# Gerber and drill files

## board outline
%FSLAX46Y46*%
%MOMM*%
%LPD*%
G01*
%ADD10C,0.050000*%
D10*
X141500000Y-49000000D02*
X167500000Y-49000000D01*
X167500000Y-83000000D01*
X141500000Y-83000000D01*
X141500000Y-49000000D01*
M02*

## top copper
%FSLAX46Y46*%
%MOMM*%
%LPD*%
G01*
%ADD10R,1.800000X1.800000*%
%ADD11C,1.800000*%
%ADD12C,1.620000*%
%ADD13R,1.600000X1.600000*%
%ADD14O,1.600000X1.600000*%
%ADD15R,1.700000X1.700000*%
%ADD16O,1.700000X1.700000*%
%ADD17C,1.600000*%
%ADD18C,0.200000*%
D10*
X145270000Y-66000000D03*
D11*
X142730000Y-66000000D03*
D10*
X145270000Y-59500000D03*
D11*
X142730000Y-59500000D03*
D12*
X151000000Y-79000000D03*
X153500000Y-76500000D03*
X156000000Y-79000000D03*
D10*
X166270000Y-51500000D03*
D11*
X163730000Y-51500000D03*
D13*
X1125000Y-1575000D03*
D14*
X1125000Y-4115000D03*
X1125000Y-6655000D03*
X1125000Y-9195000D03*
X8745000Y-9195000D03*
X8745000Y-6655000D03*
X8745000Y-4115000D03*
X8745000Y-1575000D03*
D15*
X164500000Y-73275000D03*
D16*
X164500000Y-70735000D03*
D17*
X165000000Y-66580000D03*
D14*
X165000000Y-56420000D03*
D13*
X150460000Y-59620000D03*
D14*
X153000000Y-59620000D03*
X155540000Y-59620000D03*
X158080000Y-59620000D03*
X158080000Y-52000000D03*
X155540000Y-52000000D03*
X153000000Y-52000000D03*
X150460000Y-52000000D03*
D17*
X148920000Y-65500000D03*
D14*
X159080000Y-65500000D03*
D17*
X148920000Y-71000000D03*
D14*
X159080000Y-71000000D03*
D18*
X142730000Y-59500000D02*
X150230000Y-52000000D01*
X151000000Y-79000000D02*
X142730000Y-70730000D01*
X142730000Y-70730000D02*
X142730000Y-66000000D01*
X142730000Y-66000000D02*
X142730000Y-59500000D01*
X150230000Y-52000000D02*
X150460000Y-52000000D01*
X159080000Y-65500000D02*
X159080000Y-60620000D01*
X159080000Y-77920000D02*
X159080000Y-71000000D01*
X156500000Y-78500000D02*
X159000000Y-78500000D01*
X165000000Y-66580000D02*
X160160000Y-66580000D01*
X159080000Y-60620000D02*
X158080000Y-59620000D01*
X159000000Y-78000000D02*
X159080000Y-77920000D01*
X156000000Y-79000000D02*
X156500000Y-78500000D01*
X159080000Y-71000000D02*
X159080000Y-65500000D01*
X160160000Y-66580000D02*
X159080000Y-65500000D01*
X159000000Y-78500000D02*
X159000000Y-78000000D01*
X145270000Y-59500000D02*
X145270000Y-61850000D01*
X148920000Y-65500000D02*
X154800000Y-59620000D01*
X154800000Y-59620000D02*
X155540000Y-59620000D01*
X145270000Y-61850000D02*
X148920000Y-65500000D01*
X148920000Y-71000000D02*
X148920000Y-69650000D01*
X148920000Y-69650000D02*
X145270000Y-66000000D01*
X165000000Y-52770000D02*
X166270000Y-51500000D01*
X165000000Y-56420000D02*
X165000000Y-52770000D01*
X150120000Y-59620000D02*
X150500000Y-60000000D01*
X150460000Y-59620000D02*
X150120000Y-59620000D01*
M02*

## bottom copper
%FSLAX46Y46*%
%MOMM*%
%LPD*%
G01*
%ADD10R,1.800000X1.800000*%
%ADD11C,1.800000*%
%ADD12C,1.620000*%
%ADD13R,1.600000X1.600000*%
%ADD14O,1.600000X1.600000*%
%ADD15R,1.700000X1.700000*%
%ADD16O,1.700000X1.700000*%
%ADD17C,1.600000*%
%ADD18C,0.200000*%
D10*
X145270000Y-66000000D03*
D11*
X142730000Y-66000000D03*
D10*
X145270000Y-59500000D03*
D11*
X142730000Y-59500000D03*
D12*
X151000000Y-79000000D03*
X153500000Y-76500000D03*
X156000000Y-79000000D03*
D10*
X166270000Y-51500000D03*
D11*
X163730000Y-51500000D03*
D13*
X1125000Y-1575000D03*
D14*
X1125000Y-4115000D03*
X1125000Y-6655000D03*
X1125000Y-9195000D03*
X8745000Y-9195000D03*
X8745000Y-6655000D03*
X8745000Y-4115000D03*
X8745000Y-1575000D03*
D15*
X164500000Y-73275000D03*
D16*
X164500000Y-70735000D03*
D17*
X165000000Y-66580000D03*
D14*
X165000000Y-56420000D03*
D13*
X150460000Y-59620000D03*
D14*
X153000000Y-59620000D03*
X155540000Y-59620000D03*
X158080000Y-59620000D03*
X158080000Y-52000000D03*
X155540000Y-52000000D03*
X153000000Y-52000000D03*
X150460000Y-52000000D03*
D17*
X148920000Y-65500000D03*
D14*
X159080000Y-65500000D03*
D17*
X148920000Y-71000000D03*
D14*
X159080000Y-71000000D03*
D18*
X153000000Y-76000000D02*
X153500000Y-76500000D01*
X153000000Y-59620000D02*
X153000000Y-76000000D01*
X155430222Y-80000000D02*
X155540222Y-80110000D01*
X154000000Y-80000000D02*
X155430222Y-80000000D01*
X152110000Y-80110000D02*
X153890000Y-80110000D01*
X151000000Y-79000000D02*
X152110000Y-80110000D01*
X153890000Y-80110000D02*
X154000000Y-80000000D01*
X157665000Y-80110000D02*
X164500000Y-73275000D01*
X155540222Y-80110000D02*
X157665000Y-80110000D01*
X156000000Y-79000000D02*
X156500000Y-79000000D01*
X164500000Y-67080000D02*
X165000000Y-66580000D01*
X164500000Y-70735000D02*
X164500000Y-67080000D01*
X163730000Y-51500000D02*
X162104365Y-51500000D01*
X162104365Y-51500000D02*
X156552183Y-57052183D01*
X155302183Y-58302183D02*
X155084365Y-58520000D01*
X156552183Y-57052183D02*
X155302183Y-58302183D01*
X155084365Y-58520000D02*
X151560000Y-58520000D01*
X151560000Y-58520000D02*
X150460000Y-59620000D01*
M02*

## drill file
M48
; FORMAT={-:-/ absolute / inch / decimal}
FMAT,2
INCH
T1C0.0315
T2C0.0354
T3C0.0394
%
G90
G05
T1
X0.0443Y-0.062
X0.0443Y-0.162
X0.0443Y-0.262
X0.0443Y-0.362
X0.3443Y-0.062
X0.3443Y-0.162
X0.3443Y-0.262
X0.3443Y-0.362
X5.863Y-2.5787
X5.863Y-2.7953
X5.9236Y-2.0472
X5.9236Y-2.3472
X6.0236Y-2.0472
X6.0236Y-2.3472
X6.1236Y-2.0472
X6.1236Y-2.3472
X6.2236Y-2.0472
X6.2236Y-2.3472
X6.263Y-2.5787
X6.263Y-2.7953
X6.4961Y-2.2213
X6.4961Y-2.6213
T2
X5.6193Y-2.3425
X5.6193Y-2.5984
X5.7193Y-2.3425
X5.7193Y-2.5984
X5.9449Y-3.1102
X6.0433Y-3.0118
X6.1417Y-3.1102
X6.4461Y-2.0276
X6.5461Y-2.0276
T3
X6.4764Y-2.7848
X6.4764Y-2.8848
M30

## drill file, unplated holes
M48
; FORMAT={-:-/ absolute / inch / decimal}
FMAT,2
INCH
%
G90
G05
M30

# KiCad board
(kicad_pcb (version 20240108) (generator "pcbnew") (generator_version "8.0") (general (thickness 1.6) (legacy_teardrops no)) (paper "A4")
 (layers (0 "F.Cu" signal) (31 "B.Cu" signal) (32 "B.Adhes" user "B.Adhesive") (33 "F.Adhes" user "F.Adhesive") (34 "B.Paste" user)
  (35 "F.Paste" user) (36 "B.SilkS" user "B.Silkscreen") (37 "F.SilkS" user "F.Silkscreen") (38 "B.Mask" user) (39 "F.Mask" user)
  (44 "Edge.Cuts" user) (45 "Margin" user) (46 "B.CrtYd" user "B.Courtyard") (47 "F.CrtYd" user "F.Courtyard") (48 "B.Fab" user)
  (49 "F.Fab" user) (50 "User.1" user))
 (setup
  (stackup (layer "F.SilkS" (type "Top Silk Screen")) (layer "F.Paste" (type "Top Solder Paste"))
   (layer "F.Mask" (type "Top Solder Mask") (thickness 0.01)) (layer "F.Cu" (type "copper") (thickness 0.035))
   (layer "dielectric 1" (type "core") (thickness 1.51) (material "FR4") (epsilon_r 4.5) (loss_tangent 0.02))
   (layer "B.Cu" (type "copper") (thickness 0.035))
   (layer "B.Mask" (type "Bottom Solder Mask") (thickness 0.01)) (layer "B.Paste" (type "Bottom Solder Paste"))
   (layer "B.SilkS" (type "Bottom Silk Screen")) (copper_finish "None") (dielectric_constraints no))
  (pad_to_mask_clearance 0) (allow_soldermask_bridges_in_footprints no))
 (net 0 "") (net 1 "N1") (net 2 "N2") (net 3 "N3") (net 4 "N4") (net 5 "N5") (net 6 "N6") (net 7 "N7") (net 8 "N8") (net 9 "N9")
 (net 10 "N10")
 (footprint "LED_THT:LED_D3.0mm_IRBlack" (layer "F.Cu") (at 145.27 59.5 180)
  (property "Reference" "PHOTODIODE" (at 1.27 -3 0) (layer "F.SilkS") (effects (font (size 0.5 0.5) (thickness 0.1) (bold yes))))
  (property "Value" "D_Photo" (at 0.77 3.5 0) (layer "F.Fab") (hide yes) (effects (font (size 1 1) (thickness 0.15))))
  (pad "1" thru_hole rect (at 0 0 180) (size 1.8 1.8) (drill 0.9) (layers "*.Cu" "*.Mask") (remove_unused_layers no) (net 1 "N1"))
  (pad "2" thru_hole circle (at 2.54 0 180) (size 1.8 1.8) (drill 0.9) (layers "*.Cu" "*.Mask") (remove_unused_layers no) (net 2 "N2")))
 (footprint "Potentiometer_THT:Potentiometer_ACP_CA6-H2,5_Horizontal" (layer "F.Cu") (at 151 79 90)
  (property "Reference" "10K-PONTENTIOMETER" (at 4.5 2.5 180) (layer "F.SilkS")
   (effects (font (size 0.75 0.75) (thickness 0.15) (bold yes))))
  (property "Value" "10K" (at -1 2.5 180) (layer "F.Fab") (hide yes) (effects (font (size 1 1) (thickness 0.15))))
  (pad "1" thru_hole circle (at 0 0 90) (size 1.62 1.62) (drill 0.9) (layers "*.Cu" "*.Mask") (remove_unused_layers no) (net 2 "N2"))
  (pad "2" thru_hole circle (at 2.5 2.5 90) (size 1.62 1.62) (drill 0.9) (layers "*.Cu" "*.Mask") (remove_unused_layers no) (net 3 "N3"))
  (pad "3" thru_hole circle (at 0 5 90) (size 1.62 1.62) (drill 0.9) (layers "*.Cu" "*.Mask") (remove_unused_layers no) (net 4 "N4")))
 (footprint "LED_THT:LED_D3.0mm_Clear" (layer "F.Cu") (at 145.27 66 180)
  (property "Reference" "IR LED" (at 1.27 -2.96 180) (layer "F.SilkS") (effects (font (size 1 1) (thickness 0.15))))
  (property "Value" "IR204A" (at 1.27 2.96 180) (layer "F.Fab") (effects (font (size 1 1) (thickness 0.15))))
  (pad "1" thru_hole rect (at 0 0 180) (size 1.8 1.8) (drill 0.9) (layers "*.Cu" "*.Mask") (remove_unused_layers no) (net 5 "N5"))
  (pad "2" thru_hole circle (at 2.54 0 180) (size 1.8 1.8) (drill 0.9) (layers "*.Cu" "*.Mask") (remove_unused_layers no) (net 2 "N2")))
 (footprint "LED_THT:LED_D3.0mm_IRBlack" (layer "F.Cu") (at 166.27 51.5 180)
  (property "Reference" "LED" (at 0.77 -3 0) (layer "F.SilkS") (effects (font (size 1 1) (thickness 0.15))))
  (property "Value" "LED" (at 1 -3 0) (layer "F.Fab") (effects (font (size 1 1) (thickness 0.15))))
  (pad "1" thru_hole rect (at 0 0 180) (size 1.8 1.8) (drill 0.9) (layers "*.Cu" "*.Mask") (remove_unused_layers no) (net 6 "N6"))
  (pad "2" thru_hole circle (at 2.54 0 180) (size 1.8 1.8) (drill 0.9) (layers "*.Cu" "*.Mask") (remove_unused_layers no) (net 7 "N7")))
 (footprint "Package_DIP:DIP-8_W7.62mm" (layer "F.Cu") (at 1.125 1.575)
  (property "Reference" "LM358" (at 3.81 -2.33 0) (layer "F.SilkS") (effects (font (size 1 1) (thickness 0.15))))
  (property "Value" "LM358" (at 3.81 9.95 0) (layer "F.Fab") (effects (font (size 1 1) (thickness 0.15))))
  (pad "1" thru_hole rect (at 0 0) (size 1.6 1.6) (drill 0.8) (layers "*.Cu" "*.Mask") (remove_unused_layers no))
  (pad "2" thru_hole oval (at 0 2.54) (size 1.6 1.6) (drill 0.8) (layers "*.Cu" "*.Mask") (remove_unused_layers no))
  (pad "3" thru_hole oval (at 0 5.08) (size 1.6 1.6) (drill 0.8) (layers "*.Cu" "*.Mask") (remove_unused_layers no))
  (pad "4" thru_hole oval (at 0 7.62) (size 1.6 1.6) (drill 0.8) (layers "*.Cu" "*.Mask") (remove_unused_layers no))
  (pad "5" thru_hole oval (at 7.62 7.62) (size 1.6 1.6) (drill 0.8) (layers "*.Cu" "*.Mask") (remove_unused_layers no) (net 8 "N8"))
  (pad "6" thru_hole oval (at 7.62 5.08) (size 1.6 1.6) (drill 0.8) (layers "*.Cu" "*.Mask") (remove_unused_layers no) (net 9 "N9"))
  (pad "7" thru_hole oval (at 7.62 2.54) (size 1.6 1.6) (drill 0.8) (layers "*.Cu" "*.Mask") (remove_unused_layers no) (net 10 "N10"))
  (pad "8" thru_hole oval (at 7.62 0) (size 1.6 1.6) (drill 0.8) (layers "*.Cu" "*.Mask") (remove_unused_layers no)))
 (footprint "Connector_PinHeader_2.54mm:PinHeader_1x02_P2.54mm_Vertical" (layer "F.Cu") (at 164.5 73.275 180)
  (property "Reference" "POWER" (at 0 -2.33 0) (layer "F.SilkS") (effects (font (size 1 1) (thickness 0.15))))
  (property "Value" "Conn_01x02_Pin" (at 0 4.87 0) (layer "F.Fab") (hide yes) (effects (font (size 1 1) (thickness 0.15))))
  (pad "1" thru_hole rect (at 0 0 180) (size 1.7 1.7) (drill 1) (layers "*.Cu" "*.Mask") (remove_unused_layers no) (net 2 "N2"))
  (pad "2" thru_hole oval (at 0 2.54 180) (size 1.7 1.7) (drill 1) (layers "*.Cu" "*.Mask") (remove_unused_layers no) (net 4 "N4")))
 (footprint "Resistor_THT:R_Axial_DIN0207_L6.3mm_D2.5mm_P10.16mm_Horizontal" (layer "F.Cu") (at 165 66.58 90)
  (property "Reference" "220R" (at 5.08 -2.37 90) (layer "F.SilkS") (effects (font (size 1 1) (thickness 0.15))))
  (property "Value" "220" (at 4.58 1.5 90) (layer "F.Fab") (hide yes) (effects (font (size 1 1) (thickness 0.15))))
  (pad "1" thru_hole circle (at 0 0 90) (size 1.6 1.6) (drill 0.8) (layers "*.Cu" "*.Mask") (remove_unused_layers no) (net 4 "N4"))
  (pad "2" thru_hole oval (at 10.16 0 90) (size 1.6 1.6) (drill 0.8) (layers "*.Cu" "*.Mask") (remove_unused_layers no) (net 6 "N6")))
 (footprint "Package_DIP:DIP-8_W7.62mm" (layer "F.Cu") (at 150.46 59.62 90)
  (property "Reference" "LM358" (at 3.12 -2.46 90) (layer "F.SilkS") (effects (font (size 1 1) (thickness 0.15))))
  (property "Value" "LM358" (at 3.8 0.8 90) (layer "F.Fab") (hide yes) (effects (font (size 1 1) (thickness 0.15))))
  (pad "1" thru_hole rect (at 0 0 90) (size 1.6 1.6) (drill 0.8) (layers "*.Cu" "*.Mask") (remove_unused_layers no) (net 7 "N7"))
  (pad "2" thru_hole oval (at 0 2.54 90) (size 1.6 1.6) (drill 0.8) (layers "*.Cu" "*.Mask") (remove_unused_layers no) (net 3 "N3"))
  (pad "3" thru_hole oval (at 0 5.08 90) (size 1.6 1.6) (drill 0.8) (layers "*.Cu" "*.Mask") (remove_unused_layers no) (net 1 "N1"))
  (pad "4" thru_hole oval (at 0 7.62 90) (size 1.6 1.6) (drill 0.8) (layers "*.Cu" "*.Mask") (remove_unused_layers no) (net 4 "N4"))
  (pad "5" thru_hole oval (at 7.62 7.62 90) (size 1.6 1.6) (drill 0.8) (layers "*.Cu" "*.Mask") (remove_unused_layers no))
  (pad "6" thru_hole oval (at 7.62 5.08 90) (size 1.6 1.6) (drill 0.8) (layers "*.Cu" "*.Mask") (remove_unused_layers no))
  (pad "7" thru_hole oval (at 7.62 2.54 90) (size 1.6 1.6) (drill 0.8) (layers "*.Cu" "*.Mask") (remove_unused_layers no))
  (pad "8" thru_hole oval (at 7.62 0 90) (size 1.6 1.6) (drill 0.8) (layers "*.Cu" "*.Mask") (remove_unused_layers no) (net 2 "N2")))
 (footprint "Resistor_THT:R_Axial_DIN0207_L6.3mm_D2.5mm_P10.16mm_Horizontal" (layer "F.Cu") (at 148.92 65.5)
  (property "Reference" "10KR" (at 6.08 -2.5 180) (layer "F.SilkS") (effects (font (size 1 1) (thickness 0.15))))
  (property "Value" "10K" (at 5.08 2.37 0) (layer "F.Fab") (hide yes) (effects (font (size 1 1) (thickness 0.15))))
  (pad "1" thru_hole circle (at 0 0) (size 1.6 1.6) (drill 0.8) (layers "*.Cu" "*.Mask") (remove_unused_layers no) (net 1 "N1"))
  (pad "2" thru_hole oval (at 10.16 0) (size 1.6 1.6) (drill 0.8) (layers "*.Cu" "*.Mask") (remove_unused_layers no) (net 4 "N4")))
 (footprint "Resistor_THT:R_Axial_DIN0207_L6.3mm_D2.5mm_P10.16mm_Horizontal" (layer "F.Cu") (at 148.92 71)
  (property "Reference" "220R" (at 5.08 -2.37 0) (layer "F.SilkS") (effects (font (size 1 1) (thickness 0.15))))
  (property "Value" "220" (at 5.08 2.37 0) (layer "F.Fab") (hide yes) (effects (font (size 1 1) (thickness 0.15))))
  (pad "1" thru_hole circle (at 0 0) (size 1.6 1.6) (drill 0.8) (layers "*.Cu" "*.Mask") (remove_unused_layers no) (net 5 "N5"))
  (pad "2" thru_hole oval (at 10.16 0) (size 1.6 1.6) (drill 0.8) (layers "*.Cu" "*.Mask") (remove_unused_layers no) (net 4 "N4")))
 (gr_rect (start 141.5 49) (end 167.5 83) (stroke (width 0.05) (type default)) (fill none) (layer "Edge.Cuts"))
 (segment (start 153 76) (end 153.5 76.5) (width 0.2) (layer "B.Cu") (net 3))
 (segment (start 153 59.62) (end 153 76) (width 0.2) (layer "B.Cu") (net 3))
 (segment (start 142.73 59.5) (end 150.23 52) (width 0.2) (layer "F.Cu") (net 2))
 (segment (start 151 79) (end 142.73 70.73) (width 0.2) (layer "F.Cu") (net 2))
 (segment (start 142.73 70.73) (end 142.73 66) (width 0.2) (layer "F.Cu") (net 2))
 (segment (start 142.73 66) (end 142.73 59.5) (width 0.2) (layer "F.Cu") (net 2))
 (segment (start 150.23 52) (end 150.46 52) (width 0.2) (layer "F.Cu") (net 2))
 (segment (start 155.430222 80) (end 155.540222 80.11) (width 0.2) (layer "B.Cu") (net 2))
 (segment (start 154 80) (end 155.430222 80) (width 0.2) (layer "B.Cu") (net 2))
 (segment (start 152.11 80.11) (end 153.89 80.11) (width 0.2) (layer "B.Cu") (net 2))
 (segment (start 151 79) (end 152.11 80.11) (width 0.2) (layer "B.Cu") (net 2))
 (segment (start 153.89 80.11) (end 154 80) (width 0.2) (layer "B.Cu") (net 2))
 (segment (start 157.665 80.11) (end 164.5 73.275) (width 0.2) (layer "B.Cu") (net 2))
 (segment (start 155.540222 80.11) (end 157.665 80.11) (width 0.2) (layer "B.Cu") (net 2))
 (segment (start 159.08 65.5) (end 159.08 60.62) (width 0.2) (layer "F.Cu") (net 4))
 (segment (start 159.08 77.92) (end 159.08 71) (width 0.2) (layer "F.Cu") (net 4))
 (segment (start 156.5 78.5) (end 159 78.5) (width 0.2) (layer "F.Cu") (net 4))
 (segment (start 165 66.58) (end 160.16 66.58) (width 0.2) (layer "F.Cu") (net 4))
 (segment (start 159.08 60.62) (end 158.08 59.62) (width 0.2) (layer "F.Cu") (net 4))
 (segment (start 159 78) (end 159.08 77.92) (width 0.2) (layer "F.Cu") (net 4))
 (segment (start 156 79) (end 156.5 78.5) (width 0.2) (layer "F.Cu") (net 4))
 (segment (start 159.08 71) (end 159.08 65.5) (width 0.2) (layer "F.Cu") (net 4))
 (segment (start 160.16 66.58) (end 159.08 65.5) (width 0.2) (layer "F.Cu") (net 4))
 (segment (start 159 78.5) (end 159 78) (width 0.2) (layer "F.Cu") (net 4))
 (segment (start 156 79) (end 156.5 79) (width 0.2) (layer "B.Cu") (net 4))
 (segment (start 164.5 67.08) (end 165 66.58) (width 0.2) (layer "B.Cu") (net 4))
 (segment (start 164.5 70.735) (end 164.5 67.08) (width 0.2) (layer "B.Cu") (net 4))
 (segment (start 145.27 59.5) (end 145.27 61.85) (width 0.2) (layer "F.Cu") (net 1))
 (segment (start 148.92 65.5) (end 154.8 59.62) (width 0.2) (layer "F.Cu") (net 1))
 (segment (start 154.8 59.62) (end 155.54 59.62) (width 0.2) (layer "F.Cu") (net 1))
 (segment (start 145.27 61.85) (end 148.92 65.5) (width 0.2) (layer "F.Cu") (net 1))
 (segment (start 148.92 71) (end 148.92 69.65) (width 0.2) (layer "F.Cu") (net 5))
 (segment (start 148.92 69.65) (end 145.27 66) (width 0.2) (layer "F.Cu") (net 5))
 (segment (start 165 52.77) (end 166.27 51.5) (width 0.2) (layer "F.Cu") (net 6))
 (segment (start 165 56.42) (end 165 52.77) (width 0.2) (layer "F.Cu") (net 6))
 (segment (start 150.12 59.62) (end 150.5 60) (width 0.2) (layer "F.Cu") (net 7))
 (segment (start 150.46 59.62) (end 150.12 59.62) (width 0.2) (layer "F.Cu") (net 7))
 (segment (start 163.73 51.5) (end 162.104365 51.5) (width 0.2) (layer "B.Cu") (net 7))
 (segment (start 162.104365 51.5) (end 156.552183 57.052183) (width 0.2) (layer "B.Cu") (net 7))
 (segment (start 155.302183 58.302183) (end 155.084365 58.52) (width 0.2) (layer "B.Cu") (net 7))
 (segment (start 156.552183 57.052183) (end 155.302183 58.302183) (width 0.2) (layer "B.Cu") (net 7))
 (segment (start 155.084365 58.52) (end 151.56 58.52) (width 0.2) (layer "B.Cu") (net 7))
 (segment (start 151.56 58.52) (end 150.46 59.62) (width 0.2) (layer "B.Cu") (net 7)))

